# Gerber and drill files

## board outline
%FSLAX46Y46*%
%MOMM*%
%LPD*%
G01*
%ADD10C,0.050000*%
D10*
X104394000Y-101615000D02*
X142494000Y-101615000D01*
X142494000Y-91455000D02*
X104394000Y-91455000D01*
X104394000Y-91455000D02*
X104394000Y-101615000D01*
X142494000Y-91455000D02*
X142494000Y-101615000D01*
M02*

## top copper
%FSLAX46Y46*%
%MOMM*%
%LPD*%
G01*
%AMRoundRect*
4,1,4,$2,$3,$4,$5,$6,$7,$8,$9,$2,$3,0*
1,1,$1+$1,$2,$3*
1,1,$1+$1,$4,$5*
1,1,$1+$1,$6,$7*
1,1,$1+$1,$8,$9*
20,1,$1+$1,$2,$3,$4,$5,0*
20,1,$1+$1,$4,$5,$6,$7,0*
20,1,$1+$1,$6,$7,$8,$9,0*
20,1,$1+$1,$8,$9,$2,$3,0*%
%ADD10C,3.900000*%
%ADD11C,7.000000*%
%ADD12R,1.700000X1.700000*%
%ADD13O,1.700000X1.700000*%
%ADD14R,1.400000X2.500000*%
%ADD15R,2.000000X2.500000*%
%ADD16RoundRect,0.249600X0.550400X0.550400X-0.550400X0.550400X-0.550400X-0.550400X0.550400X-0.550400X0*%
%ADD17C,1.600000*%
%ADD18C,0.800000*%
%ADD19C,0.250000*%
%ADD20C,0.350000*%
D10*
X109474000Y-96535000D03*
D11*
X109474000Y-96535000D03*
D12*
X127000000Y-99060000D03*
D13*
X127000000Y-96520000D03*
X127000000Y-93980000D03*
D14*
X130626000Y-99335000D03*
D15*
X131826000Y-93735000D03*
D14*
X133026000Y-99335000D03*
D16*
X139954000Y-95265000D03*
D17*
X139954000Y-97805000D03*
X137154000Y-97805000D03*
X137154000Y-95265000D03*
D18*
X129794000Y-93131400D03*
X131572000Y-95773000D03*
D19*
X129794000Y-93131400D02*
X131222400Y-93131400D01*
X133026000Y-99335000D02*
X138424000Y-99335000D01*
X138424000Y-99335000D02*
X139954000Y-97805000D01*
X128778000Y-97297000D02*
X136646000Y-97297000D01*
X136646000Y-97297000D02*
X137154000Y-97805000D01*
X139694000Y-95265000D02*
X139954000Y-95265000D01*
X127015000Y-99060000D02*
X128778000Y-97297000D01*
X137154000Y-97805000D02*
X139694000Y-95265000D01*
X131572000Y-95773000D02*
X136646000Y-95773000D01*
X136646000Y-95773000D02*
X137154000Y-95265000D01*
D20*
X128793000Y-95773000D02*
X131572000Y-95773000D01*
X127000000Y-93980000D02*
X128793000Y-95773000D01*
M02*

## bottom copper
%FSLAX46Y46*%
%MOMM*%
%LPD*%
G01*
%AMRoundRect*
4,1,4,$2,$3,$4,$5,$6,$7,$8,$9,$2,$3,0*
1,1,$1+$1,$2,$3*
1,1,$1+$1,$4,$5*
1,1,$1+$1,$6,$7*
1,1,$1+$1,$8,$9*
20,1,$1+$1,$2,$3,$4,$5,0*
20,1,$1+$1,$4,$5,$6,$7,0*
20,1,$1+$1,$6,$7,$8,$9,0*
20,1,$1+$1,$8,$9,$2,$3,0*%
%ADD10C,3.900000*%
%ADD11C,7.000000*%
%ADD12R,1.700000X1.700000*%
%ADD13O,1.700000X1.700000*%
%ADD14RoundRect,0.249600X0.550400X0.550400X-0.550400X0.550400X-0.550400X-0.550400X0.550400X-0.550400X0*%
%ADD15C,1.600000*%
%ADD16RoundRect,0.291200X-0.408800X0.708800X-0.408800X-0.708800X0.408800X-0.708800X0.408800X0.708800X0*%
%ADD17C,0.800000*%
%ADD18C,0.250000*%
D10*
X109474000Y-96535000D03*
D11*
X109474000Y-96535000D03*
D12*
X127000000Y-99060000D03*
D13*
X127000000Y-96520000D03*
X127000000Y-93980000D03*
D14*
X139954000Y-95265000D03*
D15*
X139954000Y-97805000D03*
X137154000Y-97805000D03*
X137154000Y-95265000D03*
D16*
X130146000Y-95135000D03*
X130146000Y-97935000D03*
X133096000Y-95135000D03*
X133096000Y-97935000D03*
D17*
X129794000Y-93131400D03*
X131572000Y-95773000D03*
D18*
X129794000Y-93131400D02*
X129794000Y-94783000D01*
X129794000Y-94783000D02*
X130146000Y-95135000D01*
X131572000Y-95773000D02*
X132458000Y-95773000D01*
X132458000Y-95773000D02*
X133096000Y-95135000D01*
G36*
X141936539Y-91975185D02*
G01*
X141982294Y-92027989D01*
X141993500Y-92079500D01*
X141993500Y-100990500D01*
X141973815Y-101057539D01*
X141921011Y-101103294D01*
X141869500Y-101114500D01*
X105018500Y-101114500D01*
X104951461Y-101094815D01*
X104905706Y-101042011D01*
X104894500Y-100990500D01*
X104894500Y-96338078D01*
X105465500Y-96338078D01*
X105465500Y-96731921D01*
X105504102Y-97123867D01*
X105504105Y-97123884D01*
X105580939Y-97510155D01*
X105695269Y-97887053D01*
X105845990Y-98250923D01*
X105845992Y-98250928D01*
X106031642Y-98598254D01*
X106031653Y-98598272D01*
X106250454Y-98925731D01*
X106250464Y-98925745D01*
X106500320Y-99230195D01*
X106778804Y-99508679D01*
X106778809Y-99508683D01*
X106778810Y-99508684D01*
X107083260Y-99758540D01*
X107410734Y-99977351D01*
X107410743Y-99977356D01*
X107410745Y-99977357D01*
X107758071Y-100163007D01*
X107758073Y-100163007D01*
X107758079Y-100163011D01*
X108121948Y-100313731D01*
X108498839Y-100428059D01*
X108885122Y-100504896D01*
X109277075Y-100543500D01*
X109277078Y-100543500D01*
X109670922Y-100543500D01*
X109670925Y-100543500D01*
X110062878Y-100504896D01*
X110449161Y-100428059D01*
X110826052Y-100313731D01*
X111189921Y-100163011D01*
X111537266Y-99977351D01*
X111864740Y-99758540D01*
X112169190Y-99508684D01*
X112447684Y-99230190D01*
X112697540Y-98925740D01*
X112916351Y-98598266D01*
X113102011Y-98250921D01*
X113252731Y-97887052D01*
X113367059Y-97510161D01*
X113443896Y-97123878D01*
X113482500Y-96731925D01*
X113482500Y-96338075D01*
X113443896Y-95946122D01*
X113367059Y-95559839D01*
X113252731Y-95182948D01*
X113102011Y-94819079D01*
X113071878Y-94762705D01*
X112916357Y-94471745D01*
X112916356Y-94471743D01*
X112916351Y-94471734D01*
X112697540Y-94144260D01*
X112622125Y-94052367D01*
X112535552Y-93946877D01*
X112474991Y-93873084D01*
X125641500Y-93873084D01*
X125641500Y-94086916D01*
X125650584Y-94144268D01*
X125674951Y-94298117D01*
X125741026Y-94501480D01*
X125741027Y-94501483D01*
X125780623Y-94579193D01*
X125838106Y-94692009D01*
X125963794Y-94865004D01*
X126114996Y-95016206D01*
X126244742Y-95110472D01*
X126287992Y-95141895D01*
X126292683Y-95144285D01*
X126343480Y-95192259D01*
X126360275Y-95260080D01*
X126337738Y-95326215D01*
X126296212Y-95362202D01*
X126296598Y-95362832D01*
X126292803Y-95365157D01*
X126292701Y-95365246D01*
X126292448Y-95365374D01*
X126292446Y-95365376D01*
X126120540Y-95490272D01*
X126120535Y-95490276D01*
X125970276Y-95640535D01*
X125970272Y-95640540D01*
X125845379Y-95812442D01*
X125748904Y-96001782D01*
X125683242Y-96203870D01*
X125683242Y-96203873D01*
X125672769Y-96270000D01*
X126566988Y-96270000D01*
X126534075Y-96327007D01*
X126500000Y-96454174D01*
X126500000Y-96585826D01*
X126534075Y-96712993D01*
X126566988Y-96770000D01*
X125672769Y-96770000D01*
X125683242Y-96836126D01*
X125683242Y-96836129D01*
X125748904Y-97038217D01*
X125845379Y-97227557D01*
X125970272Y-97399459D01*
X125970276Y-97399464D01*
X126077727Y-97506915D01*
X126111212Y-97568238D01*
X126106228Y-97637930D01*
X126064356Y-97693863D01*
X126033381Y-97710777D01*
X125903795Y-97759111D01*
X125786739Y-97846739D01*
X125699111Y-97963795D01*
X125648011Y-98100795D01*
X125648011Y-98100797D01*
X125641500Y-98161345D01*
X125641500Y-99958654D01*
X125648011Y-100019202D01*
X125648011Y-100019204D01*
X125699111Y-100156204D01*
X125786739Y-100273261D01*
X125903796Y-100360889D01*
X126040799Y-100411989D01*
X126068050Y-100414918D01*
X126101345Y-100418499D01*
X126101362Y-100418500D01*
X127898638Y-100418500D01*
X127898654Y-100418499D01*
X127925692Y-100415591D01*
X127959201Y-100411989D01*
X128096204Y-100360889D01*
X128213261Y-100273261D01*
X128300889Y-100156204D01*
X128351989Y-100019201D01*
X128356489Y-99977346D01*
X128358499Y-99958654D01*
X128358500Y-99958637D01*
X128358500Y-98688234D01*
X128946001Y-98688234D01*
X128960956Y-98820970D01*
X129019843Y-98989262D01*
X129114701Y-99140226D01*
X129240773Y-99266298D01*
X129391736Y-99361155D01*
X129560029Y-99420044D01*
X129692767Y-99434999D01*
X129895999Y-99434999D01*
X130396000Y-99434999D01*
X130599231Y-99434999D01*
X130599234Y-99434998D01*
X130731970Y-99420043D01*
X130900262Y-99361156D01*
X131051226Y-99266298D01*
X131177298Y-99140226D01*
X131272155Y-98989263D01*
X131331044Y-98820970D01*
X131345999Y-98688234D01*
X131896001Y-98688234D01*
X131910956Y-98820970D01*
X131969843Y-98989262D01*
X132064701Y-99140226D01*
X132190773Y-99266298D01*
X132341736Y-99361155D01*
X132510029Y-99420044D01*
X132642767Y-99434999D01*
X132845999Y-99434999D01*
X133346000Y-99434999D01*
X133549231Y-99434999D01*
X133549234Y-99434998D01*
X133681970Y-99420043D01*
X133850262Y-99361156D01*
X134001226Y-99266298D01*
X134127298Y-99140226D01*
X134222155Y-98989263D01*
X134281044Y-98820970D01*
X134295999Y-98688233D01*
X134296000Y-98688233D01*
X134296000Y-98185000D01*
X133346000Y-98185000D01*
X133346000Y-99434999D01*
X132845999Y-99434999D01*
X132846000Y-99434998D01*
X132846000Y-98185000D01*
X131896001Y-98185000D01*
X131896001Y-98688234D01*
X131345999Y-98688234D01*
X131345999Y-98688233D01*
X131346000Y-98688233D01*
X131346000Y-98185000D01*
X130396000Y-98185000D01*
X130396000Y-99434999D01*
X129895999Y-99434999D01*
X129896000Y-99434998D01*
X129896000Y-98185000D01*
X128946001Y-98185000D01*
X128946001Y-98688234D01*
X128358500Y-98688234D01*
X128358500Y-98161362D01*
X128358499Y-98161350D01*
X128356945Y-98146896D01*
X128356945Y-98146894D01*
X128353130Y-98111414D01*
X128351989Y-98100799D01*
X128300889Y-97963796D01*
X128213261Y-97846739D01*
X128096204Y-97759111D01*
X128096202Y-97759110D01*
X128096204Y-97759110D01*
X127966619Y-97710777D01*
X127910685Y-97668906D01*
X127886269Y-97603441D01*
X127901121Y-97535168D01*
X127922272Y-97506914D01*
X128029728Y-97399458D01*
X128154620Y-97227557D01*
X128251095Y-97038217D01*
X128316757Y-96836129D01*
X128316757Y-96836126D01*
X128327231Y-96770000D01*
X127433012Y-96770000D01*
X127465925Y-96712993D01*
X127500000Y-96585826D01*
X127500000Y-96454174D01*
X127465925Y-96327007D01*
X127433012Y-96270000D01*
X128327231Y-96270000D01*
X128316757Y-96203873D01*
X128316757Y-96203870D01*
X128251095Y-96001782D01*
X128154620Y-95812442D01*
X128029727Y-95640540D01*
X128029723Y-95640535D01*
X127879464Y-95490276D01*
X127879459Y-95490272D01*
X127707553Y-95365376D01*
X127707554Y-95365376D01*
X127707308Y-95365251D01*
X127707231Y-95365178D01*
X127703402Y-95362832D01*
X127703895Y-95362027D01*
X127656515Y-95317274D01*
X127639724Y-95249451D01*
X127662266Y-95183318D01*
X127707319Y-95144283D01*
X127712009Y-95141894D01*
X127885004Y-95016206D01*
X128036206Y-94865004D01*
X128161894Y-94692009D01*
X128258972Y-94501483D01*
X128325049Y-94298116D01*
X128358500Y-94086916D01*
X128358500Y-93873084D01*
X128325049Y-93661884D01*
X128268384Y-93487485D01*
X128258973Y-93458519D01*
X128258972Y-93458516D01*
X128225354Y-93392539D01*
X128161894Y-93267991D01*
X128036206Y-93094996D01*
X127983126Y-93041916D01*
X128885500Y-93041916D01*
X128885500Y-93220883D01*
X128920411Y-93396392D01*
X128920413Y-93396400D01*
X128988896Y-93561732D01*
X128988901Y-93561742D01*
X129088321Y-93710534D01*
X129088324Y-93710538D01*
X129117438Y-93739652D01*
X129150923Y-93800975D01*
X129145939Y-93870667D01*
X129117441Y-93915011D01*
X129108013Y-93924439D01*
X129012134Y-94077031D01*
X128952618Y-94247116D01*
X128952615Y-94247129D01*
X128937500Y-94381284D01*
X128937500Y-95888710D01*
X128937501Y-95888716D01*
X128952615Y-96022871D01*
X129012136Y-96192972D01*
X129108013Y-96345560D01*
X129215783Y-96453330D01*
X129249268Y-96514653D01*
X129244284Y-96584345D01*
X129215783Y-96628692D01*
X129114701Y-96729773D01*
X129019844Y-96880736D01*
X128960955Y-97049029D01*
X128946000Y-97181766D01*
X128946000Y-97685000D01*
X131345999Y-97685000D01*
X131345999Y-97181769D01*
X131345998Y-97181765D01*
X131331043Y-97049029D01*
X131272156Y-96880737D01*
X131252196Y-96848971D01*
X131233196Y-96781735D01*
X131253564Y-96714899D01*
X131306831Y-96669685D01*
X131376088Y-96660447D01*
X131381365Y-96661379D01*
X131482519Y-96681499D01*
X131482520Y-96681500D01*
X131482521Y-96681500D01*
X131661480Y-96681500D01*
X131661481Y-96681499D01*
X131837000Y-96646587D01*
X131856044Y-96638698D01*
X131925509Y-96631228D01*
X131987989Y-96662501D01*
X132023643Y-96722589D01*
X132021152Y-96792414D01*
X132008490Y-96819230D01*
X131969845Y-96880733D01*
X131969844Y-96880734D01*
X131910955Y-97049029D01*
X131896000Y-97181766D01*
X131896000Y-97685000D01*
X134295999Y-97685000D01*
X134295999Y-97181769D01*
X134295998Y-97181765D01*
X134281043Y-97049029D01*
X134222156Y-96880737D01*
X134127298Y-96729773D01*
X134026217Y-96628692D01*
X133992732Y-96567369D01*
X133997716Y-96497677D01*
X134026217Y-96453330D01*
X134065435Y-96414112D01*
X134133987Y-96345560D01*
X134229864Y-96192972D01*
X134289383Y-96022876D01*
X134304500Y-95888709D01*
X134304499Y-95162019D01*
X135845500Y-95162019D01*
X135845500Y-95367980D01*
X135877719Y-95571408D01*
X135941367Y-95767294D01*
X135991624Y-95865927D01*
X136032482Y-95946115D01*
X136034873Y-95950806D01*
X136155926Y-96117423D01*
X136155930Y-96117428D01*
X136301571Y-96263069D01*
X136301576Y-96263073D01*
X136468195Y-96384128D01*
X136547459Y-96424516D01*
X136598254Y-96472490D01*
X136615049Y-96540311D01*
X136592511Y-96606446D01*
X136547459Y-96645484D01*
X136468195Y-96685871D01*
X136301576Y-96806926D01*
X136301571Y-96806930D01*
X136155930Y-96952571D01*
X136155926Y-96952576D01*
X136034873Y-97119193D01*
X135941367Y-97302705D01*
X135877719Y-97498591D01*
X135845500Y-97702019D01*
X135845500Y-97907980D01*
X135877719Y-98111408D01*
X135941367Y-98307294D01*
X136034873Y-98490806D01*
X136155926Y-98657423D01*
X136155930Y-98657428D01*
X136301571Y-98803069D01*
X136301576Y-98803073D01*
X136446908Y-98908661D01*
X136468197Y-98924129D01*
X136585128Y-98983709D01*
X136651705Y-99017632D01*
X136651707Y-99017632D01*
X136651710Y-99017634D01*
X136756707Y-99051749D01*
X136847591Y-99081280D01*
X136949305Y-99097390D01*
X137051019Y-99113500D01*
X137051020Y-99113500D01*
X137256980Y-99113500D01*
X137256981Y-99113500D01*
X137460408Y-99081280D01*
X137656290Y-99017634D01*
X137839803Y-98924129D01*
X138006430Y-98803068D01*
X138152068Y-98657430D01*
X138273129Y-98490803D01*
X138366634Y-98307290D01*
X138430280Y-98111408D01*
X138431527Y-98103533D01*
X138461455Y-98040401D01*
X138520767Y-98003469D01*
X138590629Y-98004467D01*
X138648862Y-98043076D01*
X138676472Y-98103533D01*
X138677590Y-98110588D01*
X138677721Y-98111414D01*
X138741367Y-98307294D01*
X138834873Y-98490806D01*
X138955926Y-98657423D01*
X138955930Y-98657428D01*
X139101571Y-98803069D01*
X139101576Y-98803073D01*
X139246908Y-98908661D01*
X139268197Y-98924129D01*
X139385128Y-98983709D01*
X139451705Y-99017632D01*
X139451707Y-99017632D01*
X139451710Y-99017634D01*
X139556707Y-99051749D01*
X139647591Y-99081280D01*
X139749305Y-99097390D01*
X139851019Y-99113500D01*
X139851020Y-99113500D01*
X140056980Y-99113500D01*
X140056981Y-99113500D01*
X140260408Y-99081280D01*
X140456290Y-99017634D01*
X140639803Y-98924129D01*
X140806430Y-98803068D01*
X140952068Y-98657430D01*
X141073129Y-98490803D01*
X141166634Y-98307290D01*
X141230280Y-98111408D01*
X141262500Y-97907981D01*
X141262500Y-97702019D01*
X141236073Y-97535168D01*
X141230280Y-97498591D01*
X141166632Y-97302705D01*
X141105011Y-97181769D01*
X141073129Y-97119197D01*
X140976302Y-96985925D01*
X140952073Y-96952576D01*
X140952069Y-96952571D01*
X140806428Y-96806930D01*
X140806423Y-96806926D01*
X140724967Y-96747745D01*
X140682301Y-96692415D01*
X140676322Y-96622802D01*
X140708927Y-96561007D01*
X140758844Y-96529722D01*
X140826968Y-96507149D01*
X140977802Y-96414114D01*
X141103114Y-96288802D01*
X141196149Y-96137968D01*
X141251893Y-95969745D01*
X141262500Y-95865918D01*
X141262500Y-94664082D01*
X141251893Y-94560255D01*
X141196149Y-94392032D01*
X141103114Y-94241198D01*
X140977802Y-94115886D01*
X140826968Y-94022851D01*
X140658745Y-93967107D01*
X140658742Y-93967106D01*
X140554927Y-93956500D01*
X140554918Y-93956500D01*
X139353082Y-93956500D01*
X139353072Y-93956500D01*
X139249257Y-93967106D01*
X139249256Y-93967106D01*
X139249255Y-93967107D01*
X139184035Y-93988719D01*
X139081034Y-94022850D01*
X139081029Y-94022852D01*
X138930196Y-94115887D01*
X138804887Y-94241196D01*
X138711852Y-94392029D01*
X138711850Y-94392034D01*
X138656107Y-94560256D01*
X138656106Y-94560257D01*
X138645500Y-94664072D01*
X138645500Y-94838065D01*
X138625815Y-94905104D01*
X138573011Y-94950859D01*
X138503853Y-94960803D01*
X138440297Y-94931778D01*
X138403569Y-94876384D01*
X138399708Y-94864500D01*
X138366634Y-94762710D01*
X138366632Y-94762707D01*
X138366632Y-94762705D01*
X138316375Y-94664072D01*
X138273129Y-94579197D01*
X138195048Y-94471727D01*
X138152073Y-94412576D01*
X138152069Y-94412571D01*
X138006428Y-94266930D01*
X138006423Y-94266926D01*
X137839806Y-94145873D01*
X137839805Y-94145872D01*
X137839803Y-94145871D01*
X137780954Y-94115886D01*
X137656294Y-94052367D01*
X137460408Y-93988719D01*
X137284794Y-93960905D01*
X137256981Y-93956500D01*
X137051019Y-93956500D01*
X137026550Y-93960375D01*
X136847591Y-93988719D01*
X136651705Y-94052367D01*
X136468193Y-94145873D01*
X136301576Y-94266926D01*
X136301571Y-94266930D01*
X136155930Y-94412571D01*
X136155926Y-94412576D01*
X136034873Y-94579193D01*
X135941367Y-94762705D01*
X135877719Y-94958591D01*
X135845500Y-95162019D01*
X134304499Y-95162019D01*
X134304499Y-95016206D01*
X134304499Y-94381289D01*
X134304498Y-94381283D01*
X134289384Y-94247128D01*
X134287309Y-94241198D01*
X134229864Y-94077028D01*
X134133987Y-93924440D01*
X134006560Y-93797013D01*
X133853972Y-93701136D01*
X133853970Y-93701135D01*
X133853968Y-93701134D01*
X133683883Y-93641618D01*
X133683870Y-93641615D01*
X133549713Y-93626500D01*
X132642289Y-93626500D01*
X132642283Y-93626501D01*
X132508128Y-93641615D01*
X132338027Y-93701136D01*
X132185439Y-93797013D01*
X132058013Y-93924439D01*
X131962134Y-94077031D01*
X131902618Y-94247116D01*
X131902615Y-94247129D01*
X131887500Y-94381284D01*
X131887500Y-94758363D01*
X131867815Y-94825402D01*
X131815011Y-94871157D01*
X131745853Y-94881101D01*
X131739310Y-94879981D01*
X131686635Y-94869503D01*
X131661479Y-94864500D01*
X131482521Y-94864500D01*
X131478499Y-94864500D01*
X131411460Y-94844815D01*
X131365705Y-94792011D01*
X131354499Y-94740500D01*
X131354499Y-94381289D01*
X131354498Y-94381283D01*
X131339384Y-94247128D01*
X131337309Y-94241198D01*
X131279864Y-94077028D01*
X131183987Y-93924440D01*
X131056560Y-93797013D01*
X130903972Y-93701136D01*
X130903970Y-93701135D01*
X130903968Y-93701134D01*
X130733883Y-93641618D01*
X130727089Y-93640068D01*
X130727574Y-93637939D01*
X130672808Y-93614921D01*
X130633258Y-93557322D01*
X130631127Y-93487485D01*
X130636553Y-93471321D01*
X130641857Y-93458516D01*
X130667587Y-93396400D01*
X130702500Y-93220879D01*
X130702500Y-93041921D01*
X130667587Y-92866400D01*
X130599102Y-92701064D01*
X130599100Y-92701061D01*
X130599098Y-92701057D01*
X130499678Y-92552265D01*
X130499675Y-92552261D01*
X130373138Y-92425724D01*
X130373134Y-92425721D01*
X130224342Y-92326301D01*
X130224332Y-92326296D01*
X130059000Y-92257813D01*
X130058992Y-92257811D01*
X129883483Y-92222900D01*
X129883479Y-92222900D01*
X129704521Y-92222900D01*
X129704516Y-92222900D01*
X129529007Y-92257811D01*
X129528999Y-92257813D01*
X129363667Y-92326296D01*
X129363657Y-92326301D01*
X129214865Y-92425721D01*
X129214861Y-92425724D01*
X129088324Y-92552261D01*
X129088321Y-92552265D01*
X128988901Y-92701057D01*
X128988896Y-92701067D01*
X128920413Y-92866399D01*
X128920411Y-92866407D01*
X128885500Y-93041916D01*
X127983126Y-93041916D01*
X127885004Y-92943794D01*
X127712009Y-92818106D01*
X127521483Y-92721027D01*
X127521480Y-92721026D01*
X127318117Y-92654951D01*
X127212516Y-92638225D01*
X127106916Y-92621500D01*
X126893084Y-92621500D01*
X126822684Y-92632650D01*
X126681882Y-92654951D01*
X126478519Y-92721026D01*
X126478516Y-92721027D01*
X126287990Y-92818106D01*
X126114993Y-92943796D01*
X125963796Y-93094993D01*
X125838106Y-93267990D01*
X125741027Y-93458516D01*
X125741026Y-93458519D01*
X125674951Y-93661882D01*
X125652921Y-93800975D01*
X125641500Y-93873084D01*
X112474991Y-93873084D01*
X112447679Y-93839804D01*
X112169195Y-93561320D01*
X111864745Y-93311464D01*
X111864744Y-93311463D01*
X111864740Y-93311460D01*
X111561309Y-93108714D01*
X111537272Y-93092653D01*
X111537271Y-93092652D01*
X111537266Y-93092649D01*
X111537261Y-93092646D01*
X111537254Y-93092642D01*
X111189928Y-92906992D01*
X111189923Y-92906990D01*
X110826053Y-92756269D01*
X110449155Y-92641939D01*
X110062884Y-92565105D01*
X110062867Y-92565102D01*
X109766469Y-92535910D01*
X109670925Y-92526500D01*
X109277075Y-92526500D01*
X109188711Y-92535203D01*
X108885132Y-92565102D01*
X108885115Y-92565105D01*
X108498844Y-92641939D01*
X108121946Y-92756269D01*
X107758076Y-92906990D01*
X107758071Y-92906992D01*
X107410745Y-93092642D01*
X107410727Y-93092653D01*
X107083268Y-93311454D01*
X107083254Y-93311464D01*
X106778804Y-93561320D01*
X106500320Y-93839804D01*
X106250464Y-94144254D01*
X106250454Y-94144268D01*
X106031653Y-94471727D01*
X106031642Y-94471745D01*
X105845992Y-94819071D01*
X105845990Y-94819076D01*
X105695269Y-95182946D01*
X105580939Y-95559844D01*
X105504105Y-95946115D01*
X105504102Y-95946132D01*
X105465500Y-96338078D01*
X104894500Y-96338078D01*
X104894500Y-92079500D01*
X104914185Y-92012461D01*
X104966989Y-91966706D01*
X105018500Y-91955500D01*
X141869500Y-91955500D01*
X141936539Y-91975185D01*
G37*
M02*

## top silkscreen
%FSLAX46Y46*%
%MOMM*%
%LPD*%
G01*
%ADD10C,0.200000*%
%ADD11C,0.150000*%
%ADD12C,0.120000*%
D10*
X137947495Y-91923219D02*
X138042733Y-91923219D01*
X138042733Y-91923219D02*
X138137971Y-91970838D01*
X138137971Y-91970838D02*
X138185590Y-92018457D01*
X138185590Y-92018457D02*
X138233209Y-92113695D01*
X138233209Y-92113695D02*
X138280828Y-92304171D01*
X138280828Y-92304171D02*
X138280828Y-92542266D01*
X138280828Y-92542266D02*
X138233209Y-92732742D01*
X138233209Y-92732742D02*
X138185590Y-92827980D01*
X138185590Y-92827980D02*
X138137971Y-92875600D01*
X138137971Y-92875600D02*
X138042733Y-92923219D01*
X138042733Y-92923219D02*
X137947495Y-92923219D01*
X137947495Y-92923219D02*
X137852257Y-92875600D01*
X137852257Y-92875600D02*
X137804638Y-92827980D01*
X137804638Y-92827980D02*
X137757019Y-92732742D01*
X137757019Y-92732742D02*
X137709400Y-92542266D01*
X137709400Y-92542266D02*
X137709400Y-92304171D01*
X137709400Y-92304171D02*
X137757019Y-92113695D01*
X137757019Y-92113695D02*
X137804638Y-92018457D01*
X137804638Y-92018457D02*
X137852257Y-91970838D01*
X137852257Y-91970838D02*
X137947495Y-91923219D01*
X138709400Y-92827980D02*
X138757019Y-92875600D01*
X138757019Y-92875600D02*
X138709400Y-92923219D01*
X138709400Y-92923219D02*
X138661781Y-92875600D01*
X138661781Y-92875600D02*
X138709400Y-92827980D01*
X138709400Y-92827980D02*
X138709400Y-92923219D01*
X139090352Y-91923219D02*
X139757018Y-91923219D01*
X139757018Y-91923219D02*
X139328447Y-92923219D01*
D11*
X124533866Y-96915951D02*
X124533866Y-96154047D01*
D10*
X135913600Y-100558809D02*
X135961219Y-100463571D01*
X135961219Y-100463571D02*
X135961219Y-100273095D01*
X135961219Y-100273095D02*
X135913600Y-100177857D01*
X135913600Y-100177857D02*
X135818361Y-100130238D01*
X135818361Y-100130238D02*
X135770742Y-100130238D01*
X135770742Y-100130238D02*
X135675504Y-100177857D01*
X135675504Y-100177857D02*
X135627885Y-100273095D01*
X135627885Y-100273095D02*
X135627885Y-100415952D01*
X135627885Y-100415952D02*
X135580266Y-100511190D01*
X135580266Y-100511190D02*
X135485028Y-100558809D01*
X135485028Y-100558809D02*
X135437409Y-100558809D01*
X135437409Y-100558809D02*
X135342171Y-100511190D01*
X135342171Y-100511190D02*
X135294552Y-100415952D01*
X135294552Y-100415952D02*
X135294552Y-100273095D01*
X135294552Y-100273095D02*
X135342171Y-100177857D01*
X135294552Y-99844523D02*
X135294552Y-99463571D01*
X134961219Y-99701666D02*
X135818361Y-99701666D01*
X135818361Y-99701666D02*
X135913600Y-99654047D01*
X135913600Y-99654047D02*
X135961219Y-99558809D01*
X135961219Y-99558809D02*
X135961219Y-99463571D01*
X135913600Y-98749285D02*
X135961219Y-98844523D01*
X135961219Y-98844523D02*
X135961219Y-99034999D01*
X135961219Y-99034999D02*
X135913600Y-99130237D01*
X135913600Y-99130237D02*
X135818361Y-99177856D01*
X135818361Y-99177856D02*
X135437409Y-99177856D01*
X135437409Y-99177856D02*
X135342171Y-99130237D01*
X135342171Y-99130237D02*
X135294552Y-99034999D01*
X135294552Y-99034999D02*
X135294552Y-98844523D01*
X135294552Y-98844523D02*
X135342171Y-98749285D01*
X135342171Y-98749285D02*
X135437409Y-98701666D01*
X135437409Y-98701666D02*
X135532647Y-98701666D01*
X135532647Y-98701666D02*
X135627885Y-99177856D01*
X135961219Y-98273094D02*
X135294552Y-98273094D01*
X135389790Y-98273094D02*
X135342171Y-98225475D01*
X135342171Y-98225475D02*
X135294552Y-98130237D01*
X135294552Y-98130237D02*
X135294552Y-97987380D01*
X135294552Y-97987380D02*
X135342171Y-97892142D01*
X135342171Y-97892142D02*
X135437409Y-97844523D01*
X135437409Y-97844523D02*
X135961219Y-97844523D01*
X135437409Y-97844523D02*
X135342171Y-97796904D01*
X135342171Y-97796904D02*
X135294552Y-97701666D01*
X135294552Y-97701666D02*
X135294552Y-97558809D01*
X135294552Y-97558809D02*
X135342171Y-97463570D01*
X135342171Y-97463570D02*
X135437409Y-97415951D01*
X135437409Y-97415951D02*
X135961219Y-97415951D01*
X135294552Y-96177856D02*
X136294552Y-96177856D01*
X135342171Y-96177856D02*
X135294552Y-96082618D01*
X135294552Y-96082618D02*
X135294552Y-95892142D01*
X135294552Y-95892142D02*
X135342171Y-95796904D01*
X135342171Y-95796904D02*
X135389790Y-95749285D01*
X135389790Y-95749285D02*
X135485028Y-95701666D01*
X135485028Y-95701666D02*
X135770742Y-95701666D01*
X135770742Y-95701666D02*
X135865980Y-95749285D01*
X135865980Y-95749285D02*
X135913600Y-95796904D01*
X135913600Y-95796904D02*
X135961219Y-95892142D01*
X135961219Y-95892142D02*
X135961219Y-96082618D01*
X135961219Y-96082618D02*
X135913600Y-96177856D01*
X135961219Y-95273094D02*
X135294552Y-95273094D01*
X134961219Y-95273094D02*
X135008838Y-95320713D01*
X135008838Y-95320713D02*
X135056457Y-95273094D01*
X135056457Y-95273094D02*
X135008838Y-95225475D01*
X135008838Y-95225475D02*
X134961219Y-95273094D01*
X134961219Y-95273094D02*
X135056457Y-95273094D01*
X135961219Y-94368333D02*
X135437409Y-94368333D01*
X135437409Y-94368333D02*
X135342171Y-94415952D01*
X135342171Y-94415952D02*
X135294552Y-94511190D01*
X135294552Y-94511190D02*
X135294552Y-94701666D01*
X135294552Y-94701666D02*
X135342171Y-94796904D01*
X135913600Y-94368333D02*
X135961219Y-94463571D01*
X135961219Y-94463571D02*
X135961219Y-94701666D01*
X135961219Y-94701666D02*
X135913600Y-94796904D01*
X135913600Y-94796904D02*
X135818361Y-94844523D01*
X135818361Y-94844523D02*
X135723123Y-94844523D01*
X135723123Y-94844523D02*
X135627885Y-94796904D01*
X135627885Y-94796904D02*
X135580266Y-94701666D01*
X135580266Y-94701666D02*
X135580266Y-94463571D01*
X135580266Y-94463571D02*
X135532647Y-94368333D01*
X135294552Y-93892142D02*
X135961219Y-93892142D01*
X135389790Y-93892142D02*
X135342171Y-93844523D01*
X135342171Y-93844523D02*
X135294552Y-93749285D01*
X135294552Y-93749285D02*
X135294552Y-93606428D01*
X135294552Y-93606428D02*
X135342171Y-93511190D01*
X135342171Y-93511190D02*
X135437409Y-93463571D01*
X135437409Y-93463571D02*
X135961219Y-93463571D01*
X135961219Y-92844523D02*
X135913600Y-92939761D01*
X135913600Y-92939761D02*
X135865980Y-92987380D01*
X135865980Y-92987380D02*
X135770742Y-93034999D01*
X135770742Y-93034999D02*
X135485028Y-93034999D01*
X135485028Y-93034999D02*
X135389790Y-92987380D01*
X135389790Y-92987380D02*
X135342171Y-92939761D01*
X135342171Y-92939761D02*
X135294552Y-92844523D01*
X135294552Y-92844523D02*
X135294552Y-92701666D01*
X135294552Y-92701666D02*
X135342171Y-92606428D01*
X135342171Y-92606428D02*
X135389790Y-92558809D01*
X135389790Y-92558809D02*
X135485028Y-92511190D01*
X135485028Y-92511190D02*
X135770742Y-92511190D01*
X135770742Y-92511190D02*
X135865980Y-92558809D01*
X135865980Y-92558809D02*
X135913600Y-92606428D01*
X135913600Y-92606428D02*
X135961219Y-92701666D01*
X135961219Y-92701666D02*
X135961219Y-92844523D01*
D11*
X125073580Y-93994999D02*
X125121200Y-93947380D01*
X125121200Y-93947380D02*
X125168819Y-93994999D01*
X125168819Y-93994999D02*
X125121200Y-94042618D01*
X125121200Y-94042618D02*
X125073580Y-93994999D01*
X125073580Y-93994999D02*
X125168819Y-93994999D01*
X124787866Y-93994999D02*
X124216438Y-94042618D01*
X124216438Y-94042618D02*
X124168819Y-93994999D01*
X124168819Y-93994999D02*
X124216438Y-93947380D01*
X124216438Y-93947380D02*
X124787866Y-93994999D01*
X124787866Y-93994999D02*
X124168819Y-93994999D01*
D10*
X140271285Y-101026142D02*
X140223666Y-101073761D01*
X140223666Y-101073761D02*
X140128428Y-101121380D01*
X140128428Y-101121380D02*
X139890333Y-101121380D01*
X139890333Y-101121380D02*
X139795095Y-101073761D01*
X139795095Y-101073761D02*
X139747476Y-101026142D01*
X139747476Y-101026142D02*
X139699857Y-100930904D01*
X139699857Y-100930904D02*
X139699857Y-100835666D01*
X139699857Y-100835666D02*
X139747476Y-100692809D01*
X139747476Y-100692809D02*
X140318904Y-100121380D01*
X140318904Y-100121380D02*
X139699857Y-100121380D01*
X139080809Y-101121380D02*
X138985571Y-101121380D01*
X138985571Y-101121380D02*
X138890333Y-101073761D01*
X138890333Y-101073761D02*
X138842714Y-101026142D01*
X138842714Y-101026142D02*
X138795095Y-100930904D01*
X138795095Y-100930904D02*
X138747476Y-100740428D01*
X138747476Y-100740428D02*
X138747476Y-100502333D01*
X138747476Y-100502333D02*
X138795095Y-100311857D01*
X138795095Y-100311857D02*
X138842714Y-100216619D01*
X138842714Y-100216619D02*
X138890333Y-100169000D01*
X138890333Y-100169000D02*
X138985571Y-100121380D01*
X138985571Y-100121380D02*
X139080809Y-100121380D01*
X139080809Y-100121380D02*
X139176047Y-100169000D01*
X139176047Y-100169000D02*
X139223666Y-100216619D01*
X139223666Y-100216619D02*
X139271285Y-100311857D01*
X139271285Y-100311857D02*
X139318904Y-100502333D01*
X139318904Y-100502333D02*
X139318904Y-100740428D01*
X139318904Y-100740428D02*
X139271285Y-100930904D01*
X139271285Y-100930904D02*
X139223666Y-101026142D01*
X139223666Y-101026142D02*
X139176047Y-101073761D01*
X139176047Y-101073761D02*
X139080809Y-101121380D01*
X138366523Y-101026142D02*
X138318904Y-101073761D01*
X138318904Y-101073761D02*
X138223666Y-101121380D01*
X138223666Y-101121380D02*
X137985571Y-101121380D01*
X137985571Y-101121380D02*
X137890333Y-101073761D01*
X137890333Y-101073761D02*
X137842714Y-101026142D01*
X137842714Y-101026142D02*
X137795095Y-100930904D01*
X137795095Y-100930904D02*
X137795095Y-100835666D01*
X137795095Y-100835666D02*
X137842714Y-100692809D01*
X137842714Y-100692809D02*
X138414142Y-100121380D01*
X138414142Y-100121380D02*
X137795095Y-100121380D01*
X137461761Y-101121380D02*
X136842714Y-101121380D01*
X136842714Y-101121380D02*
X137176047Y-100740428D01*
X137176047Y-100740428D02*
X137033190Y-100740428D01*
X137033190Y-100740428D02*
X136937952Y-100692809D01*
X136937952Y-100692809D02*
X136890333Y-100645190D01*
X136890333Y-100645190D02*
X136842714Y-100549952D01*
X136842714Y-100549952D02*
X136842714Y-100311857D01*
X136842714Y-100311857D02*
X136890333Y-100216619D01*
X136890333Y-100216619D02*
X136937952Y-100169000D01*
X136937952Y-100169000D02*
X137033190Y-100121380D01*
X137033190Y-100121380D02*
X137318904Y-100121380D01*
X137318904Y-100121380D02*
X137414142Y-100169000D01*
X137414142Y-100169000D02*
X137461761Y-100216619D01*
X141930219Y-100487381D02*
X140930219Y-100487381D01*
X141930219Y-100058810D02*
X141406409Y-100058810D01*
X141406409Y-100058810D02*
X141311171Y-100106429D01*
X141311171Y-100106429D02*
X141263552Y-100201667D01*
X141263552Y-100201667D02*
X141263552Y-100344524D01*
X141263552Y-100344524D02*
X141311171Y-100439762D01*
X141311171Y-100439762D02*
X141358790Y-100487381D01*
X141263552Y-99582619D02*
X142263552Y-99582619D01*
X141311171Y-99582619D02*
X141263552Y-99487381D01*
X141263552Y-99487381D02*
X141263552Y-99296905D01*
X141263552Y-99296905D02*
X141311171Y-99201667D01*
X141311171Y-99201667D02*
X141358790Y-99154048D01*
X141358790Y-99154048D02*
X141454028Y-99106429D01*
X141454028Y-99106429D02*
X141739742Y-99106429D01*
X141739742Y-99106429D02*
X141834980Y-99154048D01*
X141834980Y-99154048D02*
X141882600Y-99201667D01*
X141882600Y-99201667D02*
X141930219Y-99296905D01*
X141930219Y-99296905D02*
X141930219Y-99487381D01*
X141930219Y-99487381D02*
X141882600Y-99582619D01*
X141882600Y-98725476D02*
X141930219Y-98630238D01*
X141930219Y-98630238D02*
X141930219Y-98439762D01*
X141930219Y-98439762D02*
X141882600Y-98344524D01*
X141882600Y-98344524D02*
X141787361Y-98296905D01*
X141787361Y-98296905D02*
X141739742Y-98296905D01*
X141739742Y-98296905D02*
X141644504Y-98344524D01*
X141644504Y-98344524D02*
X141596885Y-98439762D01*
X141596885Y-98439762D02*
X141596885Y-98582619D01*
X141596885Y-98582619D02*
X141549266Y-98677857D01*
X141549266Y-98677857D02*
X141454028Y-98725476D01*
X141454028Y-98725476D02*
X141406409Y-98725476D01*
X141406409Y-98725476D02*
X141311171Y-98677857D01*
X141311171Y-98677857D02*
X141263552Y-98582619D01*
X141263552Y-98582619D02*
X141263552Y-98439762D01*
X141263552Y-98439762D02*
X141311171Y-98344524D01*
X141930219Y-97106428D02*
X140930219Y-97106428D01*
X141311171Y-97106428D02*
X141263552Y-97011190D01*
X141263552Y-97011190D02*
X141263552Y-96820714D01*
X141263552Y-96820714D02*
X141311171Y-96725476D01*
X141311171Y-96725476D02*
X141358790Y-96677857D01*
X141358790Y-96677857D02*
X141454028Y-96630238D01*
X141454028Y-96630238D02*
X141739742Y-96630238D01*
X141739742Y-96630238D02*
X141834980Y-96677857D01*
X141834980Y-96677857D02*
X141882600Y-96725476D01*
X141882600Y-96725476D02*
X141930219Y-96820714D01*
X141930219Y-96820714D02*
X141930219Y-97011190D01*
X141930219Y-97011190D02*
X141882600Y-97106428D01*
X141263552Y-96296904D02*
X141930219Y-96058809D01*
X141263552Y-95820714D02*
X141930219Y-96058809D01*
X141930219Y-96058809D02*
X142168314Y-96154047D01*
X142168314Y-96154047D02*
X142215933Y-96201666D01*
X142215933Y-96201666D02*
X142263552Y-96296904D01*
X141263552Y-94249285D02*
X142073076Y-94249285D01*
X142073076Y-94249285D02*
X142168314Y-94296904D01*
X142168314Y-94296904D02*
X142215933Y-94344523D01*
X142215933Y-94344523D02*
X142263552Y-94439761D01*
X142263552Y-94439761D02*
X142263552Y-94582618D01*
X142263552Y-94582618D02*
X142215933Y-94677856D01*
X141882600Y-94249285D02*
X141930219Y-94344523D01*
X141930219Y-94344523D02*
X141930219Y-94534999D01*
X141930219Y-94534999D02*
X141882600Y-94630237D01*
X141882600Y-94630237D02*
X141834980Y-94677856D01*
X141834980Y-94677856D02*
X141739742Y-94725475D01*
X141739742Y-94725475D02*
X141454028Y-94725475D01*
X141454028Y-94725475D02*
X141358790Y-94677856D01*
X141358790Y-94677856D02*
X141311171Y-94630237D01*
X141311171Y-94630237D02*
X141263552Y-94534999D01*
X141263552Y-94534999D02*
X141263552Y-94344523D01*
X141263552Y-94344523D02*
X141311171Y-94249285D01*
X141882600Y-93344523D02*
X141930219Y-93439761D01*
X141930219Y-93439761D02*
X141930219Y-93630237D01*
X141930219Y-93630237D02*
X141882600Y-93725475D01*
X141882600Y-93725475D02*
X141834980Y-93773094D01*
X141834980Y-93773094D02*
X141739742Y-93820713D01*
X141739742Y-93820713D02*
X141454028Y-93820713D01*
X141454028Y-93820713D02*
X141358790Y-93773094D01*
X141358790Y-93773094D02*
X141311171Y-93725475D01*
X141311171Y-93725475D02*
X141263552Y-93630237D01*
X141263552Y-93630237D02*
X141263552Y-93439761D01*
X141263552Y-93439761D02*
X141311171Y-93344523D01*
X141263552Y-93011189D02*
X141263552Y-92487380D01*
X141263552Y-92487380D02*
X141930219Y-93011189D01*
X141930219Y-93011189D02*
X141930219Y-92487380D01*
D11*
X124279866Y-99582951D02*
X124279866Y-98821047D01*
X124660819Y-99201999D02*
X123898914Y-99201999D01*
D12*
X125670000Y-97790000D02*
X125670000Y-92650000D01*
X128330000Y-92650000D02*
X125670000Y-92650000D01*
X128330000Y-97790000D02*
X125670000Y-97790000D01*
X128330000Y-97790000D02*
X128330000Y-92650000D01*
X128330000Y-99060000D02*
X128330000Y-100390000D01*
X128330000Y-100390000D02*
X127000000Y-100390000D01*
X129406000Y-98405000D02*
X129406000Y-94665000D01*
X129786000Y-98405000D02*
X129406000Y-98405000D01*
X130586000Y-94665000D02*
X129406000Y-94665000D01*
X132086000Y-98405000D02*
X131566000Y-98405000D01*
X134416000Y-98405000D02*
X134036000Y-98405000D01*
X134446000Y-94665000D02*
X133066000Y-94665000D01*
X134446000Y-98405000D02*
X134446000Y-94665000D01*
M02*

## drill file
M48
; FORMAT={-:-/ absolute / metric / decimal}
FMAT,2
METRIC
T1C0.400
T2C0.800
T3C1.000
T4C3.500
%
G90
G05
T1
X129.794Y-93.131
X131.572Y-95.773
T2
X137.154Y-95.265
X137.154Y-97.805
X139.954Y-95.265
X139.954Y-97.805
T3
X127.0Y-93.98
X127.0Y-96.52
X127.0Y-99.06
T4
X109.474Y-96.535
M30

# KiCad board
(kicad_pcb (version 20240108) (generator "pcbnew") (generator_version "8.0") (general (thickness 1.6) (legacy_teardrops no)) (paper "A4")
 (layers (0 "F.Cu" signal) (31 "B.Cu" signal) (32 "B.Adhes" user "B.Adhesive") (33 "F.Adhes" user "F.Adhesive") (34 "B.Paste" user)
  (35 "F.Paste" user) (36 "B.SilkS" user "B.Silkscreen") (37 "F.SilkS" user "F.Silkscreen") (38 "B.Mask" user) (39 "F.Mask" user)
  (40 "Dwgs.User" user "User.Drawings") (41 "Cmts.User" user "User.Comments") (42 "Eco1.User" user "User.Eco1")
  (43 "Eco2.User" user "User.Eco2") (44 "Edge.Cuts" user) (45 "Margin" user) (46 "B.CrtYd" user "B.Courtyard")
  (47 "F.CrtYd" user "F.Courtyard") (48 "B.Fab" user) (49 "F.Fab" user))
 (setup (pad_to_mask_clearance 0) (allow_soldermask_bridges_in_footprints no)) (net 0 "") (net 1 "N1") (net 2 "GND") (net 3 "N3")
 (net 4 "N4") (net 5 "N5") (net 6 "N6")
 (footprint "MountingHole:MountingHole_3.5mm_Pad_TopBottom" (layer "F.Cu") (at 109.474 96.535)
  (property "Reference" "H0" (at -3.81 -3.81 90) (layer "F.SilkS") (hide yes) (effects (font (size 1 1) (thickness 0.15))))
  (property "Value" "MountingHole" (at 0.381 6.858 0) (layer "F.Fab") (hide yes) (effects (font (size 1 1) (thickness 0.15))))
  (pad "1" thru_hole circle (at 0 0) (size 3.9 3.9) (drill 3.5) (layers "*.Cu" "*.Mask") (remove_unused_layers no))
  (pad "1" connect circle (at 0 0) (size 7 7) (layers "F.Cu" "F.Mask"))
  (pad "1" connect circle (at 0 0) (size 7 7) (layers "B.Cu" "B.Mask")))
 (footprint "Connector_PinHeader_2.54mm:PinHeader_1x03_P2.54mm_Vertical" (layer "F.Cu") (at 127 99.06 180)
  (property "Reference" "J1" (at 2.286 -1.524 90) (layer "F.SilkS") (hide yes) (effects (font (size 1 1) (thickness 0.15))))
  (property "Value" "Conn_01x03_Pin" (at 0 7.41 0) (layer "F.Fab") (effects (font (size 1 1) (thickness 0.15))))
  (fp_line (start 1.33 1.27) (end 1.33 6.41) (stroke (width 0.12) (type solid)) (layer "F.SilkS"))
  (fp_line (start -1.33 6.41) (end 1.33 6.41) (stroke (width 0.12) (type solid)) (layer "F.SilkS"))
  (fp_line (start -1.33 1.27) (end 1.33 1.27) (stroke (width 0.12) (type solid)) (layer "F.SilkS"))
  (fp_line (start -1.33 1.27) (end -1.33 6.41) (stroke (width 0.12) (type solid)) (layer "F.SilkS"))
  (fp_line (start -1.33 0) (end -1.33 -1.33) (stroke (width 0.12) (type solid)) (layer "F.SilkS"))
  (fp_line (start -1.33 -1.33) (end 0 -1.33) (stroke (width 0.12) (type solid)) (layer "F.SilkS"))
  (pad "1" thru_hole rect (at 0 0 180) (size 1.7 1.7) (drill 1) (layers "*.Cu" "*.Mask") (remove_unused_layers no) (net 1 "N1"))
  (pad "2" thru_hole oval (at 0 2.54 180) (size 1.7 1.7) (drill 1) (layers "*.Cu" "*.Mask") (remove_unused_layers no) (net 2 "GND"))
  (pad "3" thru_hole oval (at 0 5.08 180) (size 1.7 1.7) (drill 1) (layers "*.Cu" "*.Mask") (remove_unused_layers no) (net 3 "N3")))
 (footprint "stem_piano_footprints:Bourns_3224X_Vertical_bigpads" (layer "F.Cu") (at 131.826 96.535 180)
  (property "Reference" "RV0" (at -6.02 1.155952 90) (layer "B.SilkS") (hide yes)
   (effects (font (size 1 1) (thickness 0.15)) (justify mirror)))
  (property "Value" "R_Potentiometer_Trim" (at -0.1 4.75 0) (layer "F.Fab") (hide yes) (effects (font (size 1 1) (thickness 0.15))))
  (fp_line (start 2.42 -1.87) (end 2.42 1.87) (stroke (width 0.12) (type solid)) (layer "F.SilkS"))
  (fp_line (start 2.04 -1.87) (end 2.42 -1.87) (stroke (width 0.12) (type solid)) (layer "F.SilkS"))
  (fp_line (start 1.24 1.87) (end 2.42 1.87) (stroke (width 0.12) (type solid)) (layer "F.SilkS"))
  (fp_line (start -0.26 -1.87) (end 0.26 -1.87) (stroke (width 0.12) (type solid)) (layer "F.SilkS"))
  (fp_line (start -2.59 -1.87) (end -2.21 -1.87) (stroke (width 0.12) (type solid)) (layer "F.SilkS"))
  (fp_line (start -2.62 1.87) (end -1.24 1.87) (stroke (width 0.12) (type solid)) (layer "F.SilkS"))
  (fp_line (start -2.62 -1.87) (end -2.62 1.87) (stroke (width 0.12) (type solid)) (layer "F.SilkS"))
  (pad "1" smd rect (at 1.2 -2.8 180) (size 1.4 2.5) (layers "F.Cu" "F.Paste" "F.Mask") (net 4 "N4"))
  (pad "2" smd rect (at 0 2.8 180) (size 2 2.5) (layers "F.Cu" "F.Paste" "F.Mask") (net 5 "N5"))
  (pad "3" smd rect (at -1.2 -2.8 180) (size 1.4 2.5) (layers "F.Cu" "F.Paste" "F.Mask") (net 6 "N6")))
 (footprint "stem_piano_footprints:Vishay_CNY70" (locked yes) (layer "B.Cu") (at 139.954 95.265 180)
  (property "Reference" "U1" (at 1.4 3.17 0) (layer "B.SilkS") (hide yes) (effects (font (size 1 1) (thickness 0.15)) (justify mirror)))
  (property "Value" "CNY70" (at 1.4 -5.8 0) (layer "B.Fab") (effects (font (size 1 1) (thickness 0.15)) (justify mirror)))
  (pad "1" thru_hole roundrect (at 0 0 180) (size 1.6 1.6) (drill 0.8) (layers "*.Cu" "*.Mask") (remove_unused_layers no)
   (roundrect_rratio 0.156) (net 1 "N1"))
  (pad "2" thru_hole circle (at 0 -2.54 180) (size 1.6 1.6) (drill 0.8) (layers "*.Cu" "*.Mask") (remove_unused_layers no) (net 6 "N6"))
  (pad "3" thru_hole circle (at 2.8 -2.54 180) (size 1.6 1.6) (drill 0.8) (layers "*.Cu" "*.Mask") (remove_unused_layers no) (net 1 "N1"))
  (pad "4" thru_hole circle (at 2.8 0 180) (size 1.6 1.6) (drill 0.8) (layers "*.Cu" "*.Mask") (remove_unused_layers no) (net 3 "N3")))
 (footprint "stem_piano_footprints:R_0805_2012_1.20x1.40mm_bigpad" (layer "B.Cu") (at 130.146 96.535 -90)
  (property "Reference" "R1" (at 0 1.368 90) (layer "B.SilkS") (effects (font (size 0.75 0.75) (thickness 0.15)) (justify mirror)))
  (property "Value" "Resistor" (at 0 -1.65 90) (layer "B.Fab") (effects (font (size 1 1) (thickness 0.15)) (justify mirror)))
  (pad "1" smd roundrect (at -1.4 0 270) (size 2 1.4) (layers "B.Cu" "B.Paste" "B.Mask") (roundrect_rratio 0.208) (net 5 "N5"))
  (pad "2" smd roundrect (at 1.4 0 270) (size 2 1.4) (layers "B.Cu" "B.Paste" "B.Mask") (roundrect_rratio 0.208) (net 2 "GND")))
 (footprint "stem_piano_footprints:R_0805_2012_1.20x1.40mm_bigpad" (layer "B.Cu") (at 133.096 96.535 -90)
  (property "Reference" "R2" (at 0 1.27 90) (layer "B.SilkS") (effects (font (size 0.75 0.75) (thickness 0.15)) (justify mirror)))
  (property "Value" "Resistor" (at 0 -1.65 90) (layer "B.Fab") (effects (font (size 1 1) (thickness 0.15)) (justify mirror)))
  (pad "1" smd roundrect (at -1.4 0 270) (size 2 1.4) (layers "B.Cu" "B.Paste" "B.Mask") (roundrect_rratio 0.208) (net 3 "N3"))
  (pad "2" smd roundrect (at 1.4 0 270) (size 2 1.4) (layers "B.Cu" "B.Paste" "B.Mask") (roundrect_rratio 0.208) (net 2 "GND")))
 (gr_line (start 104.394 101.615) (end 142.494 101.615) (stroke (width 0.05) (type solid)) (layer "Edge.Cuts"))
 (gr_line (start 142.494 91.455) (end 104.394 91.455) (stroke (width 0.05) (type solid)) (layer "Edge.Cuts"))
 (gr_line (start 104.394 91.455) (end 104.394 101.615) (stroke (width 0.05) (type solid)) (layer "Edge.Cuts"))
 (gr_line (start 142.494 91.455) (end 142.494 101.615) (stroke (width 0.05) (type solid)) (layer "Edge.Cuts"))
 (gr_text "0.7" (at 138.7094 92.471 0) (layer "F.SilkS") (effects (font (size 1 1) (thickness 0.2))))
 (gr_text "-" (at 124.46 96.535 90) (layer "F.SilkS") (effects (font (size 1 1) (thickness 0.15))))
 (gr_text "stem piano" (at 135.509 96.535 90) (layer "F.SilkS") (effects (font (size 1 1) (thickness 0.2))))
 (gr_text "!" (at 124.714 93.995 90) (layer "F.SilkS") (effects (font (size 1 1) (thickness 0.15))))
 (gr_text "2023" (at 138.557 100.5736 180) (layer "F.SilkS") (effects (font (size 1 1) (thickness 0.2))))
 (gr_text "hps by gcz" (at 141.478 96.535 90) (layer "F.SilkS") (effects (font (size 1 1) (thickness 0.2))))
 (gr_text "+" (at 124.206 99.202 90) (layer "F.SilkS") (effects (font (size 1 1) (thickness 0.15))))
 (segment (start 129.794 93.1314) (end 131.2224 93.1314) (width 0.25) (layer "F.Cu") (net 5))
 (via (at 129.794 93.1314) (size 0.8) (drill 0.4) (layers "F.Cu" "B.Cu") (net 5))
 (segment (start 129.794 93.1314) (end 129.794 94.783) (width 0.25) (layer "B.Cu") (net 5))
 (segment (start 129.794 94.783) (end 130.146 95.135) (width 0.25) (layer "B.Cu") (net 5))
 (segment (start 133.026 99.335) (end 138.424 99.335) (width 0.25) (layer "F.Cu") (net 6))
 (segment (start 138.424 99.335) (end 139.954 97.805) (width 0.25) (layer "F.Cu") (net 6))
 (segment (start 128.778 97.297) (end 136.646 97.297) (width 0.25) (layer "F.Cu") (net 1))
 (segment (start 136.646 97.297) (end 137.154 97.805) (width 0.25) (layer "F.Cu") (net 1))
 (segment (start 139.694 95.265) (end 139.954 95.265) (width 0.25) (layer "F.Cu") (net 1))
 (segment (start 127.015 99.06) (end 128.778 97.297) (width 0.25) (layer "F.Cu") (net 1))
 (segment (start 137.154 97.805) (end 139.694 95.265) (width 0.25) (layer "F.Cu") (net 1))
 (segment (start 131.572 95.773) (end 136.646 95.773) (width 0.25) (layer "F.Cu") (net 3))
 (segment (start 136.646 95.773) (end 137.154 95.265) (width 0.25) (layer "F.Cu") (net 3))
 (segment (start 128.793 95.773) (end 131.572 95.773) (width 0.35) (layer "F.Cu") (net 3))
 (segment (start 127 93.98) (end 128.793 95.773) (width 0.35) (layer "F.Cu") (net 3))
 (via (at 131.572 95.773) (size 0.8) (drill 0.4) (layers "F.Cu" "B.Cu") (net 3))
 (segment (start 131.572 95.773) (end 132.458 95.773) (width 0.25) (layer "B.Cu") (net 3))
 (segment (start 132.458 95.773) (end 133.096 95.135) (width 0.25) (layer "B.Cu") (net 3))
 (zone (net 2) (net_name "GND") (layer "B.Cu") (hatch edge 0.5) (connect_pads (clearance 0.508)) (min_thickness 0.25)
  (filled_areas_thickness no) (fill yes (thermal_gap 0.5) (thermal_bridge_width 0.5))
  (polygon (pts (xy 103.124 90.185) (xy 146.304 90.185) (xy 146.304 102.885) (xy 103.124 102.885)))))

